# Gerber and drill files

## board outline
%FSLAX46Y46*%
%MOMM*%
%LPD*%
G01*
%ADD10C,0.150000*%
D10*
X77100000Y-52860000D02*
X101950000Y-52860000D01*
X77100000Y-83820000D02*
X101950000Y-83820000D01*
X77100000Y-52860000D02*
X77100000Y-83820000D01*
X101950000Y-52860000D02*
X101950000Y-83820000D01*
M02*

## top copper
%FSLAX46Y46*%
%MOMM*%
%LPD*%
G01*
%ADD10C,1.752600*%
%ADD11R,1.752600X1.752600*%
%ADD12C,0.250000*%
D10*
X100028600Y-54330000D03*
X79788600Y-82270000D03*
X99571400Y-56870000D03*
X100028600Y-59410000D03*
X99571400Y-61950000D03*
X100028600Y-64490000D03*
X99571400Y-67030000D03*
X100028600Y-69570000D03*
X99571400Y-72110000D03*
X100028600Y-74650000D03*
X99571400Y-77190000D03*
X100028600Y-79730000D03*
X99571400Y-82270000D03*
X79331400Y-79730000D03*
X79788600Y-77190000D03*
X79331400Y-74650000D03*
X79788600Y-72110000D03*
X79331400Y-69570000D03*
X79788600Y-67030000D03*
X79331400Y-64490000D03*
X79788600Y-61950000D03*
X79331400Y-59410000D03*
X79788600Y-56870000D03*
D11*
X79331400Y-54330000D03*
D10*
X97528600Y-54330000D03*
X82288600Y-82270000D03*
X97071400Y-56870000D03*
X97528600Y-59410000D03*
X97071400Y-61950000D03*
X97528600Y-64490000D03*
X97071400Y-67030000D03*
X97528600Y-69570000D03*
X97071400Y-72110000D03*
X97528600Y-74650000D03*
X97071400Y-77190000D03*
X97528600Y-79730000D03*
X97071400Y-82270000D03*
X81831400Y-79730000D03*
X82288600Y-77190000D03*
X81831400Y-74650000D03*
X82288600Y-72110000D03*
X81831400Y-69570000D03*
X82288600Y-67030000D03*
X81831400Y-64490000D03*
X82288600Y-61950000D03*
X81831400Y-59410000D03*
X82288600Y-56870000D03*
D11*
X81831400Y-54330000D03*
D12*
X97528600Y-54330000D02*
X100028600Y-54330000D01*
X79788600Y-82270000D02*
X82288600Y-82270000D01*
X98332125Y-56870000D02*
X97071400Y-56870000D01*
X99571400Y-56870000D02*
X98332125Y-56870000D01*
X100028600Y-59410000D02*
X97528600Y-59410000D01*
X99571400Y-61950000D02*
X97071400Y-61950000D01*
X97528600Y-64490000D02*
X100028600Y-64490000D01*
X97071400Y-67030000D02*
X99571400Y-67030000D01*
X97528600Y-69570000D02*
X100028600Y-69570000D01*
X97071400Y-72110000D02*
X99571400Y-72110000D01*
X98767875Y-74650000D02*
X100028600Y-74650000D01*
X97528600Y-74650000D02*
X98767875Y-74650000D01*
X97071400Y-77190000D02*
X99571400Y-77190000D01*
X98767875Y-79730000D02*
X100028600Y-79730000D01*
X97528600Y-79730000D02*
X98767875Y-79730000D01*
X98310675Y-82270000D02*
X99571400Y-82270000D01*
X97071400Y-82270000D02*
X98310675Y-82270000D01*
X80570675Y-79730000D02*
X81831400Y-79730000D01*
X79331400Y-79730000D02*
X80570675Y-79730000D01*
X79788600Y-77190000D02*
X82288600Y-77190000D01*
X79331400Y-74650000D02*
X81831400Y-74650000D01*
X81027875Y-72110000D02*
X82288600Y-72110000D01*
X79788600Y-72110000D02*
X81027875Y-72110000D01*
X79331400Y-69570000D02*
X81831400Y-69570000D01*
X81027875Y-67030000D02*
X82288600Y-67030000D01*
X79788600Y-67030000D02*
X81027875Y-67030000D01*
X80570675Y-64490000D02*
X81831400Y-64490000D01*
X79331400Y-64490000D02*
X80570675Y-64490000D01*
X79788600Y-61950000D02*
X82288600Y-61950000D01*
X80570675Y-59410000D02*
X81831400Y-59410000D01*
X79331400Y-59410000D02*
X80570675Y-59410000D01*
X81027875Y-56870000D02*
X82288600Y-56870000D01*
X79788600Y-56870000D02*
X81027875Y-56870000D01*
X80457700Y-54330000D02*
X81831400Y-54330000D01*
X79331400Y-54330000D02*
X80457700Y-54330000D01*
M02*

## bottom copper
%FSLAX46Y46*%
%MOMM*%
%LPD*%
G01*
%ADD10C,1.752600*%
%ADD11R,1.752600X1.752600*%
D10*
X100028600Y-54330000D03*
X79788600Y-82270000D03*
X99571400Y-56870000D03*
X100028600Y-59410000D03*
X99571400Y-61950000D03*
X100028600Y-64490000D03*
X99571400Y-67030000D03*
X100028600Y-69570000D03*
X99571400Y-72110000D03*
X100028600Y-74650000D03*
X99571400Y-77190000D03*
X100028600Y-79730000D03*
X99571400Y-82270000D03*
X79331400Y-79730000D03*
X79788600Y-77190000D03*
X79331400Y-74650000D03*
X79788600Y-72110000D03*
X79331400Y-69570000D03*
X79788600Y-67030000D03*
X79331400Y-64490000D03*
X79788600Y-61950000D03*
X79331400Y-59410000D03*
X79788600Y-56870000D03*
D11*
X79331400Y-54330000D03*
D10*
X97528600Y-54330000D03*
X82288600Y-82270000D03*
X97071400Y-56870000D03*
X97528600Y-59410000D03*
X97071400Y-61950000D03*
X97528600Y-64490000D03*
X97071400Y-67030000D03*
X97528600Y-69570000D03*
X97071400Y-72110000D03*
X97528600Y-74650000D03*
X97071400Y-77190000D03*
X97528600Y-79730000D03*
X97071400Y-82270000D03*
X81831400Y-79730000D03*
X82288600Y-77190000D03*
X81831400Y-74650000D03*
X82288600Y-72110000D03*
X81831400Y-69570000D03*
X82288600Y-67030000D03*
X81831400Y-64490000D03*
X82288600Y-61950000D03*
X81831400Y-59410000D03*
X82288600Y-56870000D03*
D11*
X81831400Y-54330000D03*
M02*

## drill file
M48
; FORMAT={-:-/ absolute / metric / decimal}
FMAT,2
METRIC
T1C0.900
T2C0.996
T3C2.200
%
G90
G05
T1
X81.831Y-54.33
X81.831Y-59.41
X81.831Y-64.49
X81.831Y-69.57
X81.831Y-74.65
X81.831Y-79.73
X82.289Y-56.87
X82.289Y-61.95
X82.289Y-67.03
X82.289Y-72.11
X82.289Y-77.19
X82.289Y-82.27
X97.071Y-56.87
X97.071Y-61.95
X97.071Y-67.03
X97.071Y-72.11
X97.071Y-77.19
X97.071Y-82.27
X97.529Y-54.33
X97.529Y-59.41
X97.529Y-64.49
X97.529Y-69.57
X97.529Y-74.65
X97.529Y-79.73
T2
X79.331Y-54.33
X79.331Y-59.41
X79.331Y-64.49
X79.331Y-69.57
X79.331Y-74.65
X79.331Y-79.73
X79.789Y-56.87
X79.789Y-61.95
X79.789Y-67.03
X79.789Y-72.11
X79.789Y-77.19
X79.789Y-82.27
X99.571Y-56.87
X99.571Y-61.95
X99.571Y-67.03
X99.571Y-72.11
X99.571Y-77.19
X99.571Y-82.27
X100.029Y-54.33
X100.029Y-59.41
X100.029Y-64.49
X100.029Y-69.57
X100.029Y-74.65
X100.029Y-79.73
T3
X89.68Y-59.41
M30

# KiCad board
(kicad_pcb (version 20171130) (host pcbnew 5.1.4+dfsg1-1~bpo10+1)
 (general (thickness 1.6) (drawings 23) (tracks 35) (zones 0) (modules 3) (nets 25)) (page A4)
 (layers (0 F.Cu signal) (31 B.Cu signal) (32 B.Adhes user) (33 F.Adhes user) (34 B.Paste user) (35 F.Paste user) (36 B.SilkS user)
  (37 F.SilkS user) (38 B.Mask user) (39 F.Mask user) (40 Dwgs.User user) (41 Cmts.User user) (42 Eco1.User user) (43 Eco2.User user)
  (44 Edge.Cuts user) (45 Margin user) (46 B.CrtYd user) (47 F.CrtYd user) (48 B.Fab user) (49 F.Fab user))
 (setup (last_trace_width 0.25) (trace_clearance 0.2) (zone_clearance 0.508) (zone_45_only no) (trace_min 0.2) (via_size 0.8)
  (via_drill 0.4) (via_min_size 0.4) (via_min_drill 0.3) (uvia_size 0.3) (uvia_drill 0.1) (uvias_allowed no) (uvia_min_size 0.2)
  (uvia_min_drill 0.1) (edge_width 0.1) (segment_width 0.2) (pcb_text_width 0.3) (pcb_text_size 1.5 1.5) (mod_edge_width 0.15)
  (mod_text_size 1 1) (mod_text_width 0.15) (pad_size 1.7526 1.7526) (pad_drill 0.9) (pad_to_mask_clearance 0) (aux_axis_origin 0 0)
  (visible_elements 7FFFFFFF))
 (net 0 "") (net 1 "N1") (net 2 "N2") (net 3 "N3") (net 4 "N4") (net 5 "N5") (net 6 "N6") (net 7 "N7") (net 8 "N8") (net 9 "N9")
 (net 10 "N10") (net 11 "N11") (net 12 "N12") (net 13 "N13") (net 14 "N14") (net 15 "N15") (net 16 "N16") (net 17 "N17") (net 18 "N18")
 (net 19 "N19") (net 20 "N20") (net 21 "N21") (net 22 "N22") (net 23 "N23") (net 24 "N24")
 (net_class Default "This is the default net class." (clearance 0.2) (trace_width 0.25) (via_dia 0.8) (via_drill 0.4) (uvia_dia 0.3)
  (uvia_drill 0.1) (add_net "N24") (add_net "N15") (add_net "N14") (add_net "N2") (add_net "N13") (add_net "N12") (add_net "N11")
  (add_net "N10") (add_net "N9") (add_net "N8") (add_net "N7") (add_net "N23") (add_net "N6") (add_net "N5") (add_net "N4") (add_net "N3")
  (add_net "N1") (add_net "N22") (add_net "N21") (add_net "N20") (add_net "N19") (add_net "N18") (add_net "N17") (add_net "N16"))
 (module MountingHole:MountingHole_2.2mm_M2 (layer F.Cu) (at 89.68 59.41)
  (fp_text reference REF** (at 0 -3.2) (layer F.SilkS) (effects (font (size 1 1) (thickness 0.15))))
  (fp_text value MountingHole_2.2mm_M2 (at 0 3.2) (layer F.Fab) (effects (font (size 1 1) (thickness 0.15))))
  (pad 1 np_thru_hole circle (at 0 0) (size 2.2 2.2) (drill 2.2) (layers *.Cu *.Mask)))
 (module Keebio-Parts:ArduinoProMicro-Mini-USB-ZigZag (layer F.Cu) (at 89.68 68.3 270)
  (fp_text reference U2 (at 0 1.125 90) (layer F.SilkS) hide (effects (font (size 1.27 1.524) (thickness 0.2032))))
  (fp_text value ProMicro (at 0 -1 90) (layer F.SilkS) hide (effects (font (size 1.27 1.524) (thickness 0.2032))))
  (pad 24 thru_hole circle (at -13.97 -10.3486 270) (size 1.7526 1.7526) (drill 0.9961) (layers *.Cu *.SilkS *.Mask) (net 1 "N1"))
  (pad 12 thru_hole circle (at 13.97 9.8914 270) (size 1.7526 1.7526) (drill 0.9961) (layers *.Cu *.SilkS *.Mask) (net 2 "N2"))
  (pad 23 thru_hole circle (at -11.43 -9.8914 270) (size 1.7526 1.7526) (drill 0.9961) (layers *.Cu *.SilkS *.Mask) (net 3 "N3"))
  (pad 22 thru_hole circle (at -8.89 -10.3486 270) (size 1.7526 1.7526) (drill 0.9961) (layers *.Cu *.SilkS *.Mask) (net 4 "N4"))
  (pad 21 thru_hole circle (at -6.35 -9.8914 270) (size 1.7526 1.7526) (drill 0.9961) (layers *.Cu *.SilkS *.Mask) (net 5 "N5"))
  (pad 20 thru_hole circle (at -3.81 -10.3486 270) (size 1.7526 1.7526) (drill 0.9961) (layers *.Cu *.SilkS *.Mask) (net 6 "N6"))
  (pad 19 thru_hole circle (at -1.27 -9.8914 270) (size 1.7526 1.7526) (drill 0.9961) (layers *.Cu *.SilkS *.Mask) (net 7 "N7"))
  (pad 18 thru_hole circle (at 1.27 -10.3486 270) (size 1.7526 1.7526) (drill 0.9961) (layers *.Cu *.SilkS *.Mask) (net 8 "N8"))
  (pad 17 thru_hole circle (at 3.81 -9.8914 270) (size 1.7526 1.7526) (drill 0.9961) (layers *.Cu *.SilkS *.Mask) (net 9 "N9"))
  (pad 16 thru_hole circle (at 6.35 -10.3486 270) (size 1.7526 1.7526) (drill 0.9961) (layers *.Cu *.SilkS *.Mask) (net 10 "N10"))
  (pad 15 thru_hole circle (at 8.89 -9.8914 270) (size 1.7526 1.7526) (drill 0.9961) (layers *.Cu *.SilkS *.Mask) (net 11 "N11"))
  (pad 14 thru_hole circle (at 11.43 -10.3486 270) (size 1.7526 1.7526) (drill 0.9961) (layers *.Cu *.SilkS *.Mask) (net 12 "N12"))
  (pad 13 thru_hole circle (at 13.97 -9.8914 270) (size 1.7526 1.7526) (drill 0.9961) (layers *.Cu *.SilkS *.Mask) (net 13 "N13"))
  (pad 11 thru_hole circle (at 11.43 10.3486 270) (size 1.7526 1.7526) (drill 0.9961) (layers *.Cu *.SilkS *.Mask) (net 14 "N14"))
  (pad 10 thru_hole circle (at 8.89 9.8914 270) (size 1.7526 1.7526) (drill 0.9961) (layers *.Cu *.SilkS *.Mask) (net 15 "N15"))
  (pad 9 thru_hole circle (at 6.35 10.3486 270) (size 1.7526 1.7526) (drill 0.9961) (layers *.Cu *.SilkS *.Mask) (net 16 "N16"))
  (pad 8 thru_hole circle (at 3.81 9.8914 270) (size 1.7526 1.7526) (drill 0.9961) (layers *.Cu *.SilkS *.Mask) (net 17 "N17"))
  (pad 7 thru_hole circle (at 1.27 10.3486 270) (size 1.7526 1.7526) (drill 0.9961) (layers *.Cu *.SilkS *.Mask) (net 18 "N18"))
  (pad 6 thru_hole circle (at -1.27 9.8914 270) (size 1.7526 1.7526) (drill 0.9961) (layers *.Cu *.SilkS *.Mask) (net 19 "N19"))
  (pad 5 thru_hole circle (at -3.81 10.3486 270) (size 1.7526 1.7526) (drill 0.9961) (layers *.Cu *.SilkS *.Mask) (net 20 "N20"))
  (pad 4 thru_hole circle (at -6.35 9.8914 270) (size 1.7526 1.7526) (drill 0.9961) (layers *.Cu *.SilkS *.Mask) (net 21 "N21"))
  (pad 3 thru_hole circle (at -8.89 10.3486 270) (size 1.7526 1.7526) (drill 0.9961) (layers *.Cu *.SilkS *.Mask) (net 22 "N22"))
  (pad 2 thru_hole circle (at -11.43 9.8914 270) (size 1.7526 1.7526) (drill 0.9961) (layers *.Cu *.SilkS *.Mask) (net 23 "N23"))
  (pad 1 thru_hole rect (at -13.97 10.3486 270) (size 1.7526 1.7526) (drill 0.9961) (layers *.Cu *.SilkS *.Mask) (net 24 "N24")))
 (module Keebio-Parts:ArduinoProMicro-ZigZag (layer F.Cu) (at 89.68 68.3 270)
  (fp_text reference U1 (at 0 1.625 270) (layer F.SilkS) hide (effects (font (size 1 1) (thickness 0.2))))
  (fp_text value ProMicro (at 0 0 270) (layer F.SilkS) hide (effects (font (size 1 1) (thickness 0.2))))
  (pad 24 thru_hole circle (at -13.97 -7.8486 270) (size 1.7526 1.7526) (drill 0.9) (layers *.Cu *.SilkS *.Mask) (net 1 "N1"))
  (pad 12 thru_hole circle (at 13.97 7.3914 270) (size 1.7526 1.7526) (drill 0.9) (layers *.Cu *.SilkS *.Mask) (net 2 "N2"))
  (pad 23 thru_hole circle (at -11.43 -7.3914 270) (size 1.7526 1.7526) (drill 0.9) (layers *.Cu *.SilkS *.Mask) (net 3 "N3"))
  (pad 22 thru_hole circle (at -8.89 -7.8486 270) (size 1.7526 1.7526) (drill 0.9) (layers *.Cu *.SilkS *.Mask) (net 4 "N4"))
  (pad 21 thru_hole circle (at -6.35 -7.3914 270) (size 1.7526 1.7526) (drill 0.9) (layers *.Cu *.SilkS *.Mask) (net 5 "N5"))
  (pad 20 thru_hole circle (at -3.81 -7.8486 270) (size 1.7526 1.7526) (drill 0.9) (layers *.Cu *.SilkS *.Mask) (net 6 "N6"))
  (pad 19 thru_hole circle (at -1.27 -7.3914 270) (size 1.7526 1.7526) (drill 0.9) (layers *.Cu *.SilkS *.Mask) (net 7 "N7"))
  (pad 18 thru_hole circle (at 1.27 -7.8486 270) (size 1.7526 1.7526) (drill 0.9) (layers *.Cu *.SilkS *.Mask) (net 8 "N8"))
  (pad 17 thru_hole circle (at 3.81 -7.3914 270) (size 1.7526 1.7526) (drill 0.9) (layers *.Cu *.SilkS *.Mask) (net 9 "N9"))
  (pad 16 thru_hole circle (at 6.35 -7.8486 270) (size 1.7526 1.7526) (drill 0.9) (layers *.Cu *.SilkS *.Mask) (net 10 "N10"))
  (pad 15 thru_hole circle (at 8.89 -7.3914 270) (size 1.7526 1.7526) (drill 0.9) (layers *.Cu *.SilkS *.Mask) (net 11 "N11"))
  (pad 14 thru_hole circle (at 11.43 -7.8486 270) (size 1.7526 1.7526) (drill 0.9) (layers *.Cu *.SilkS *.Mask) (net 12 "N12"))
  (pad 13 thru_hole circle (at 13.97 -7.3914 270) (size 1.7526 1.7526) (drill 0.9) (layers *.Cu *.SilkS *.Mask) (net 13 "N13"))
  (pad 11 thru_hole circle (at 11.43 7.8486 270) (size 1.7526 1.7526) (drill 0.9) (layers *.Cu *.SilkS *.Mask) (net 14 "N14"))
  (pad 10 thru_hole circle (at 8.89 7.3914 270) (size 1.7526 1.7526) (drill 0.9) (layers *.Cu *.SilkS *.Mask) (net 15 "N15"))
  (pad 9 thru_hole circle (at 6.35 7.8486 270) (size 1.7526 1.7526) (drill 0.9) (layers *.Cu *.SilkS *.Mask) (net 16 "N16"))
  (pad 8 thru_hole circle (at 3.81 7.3914 270) (size 1.7526 1.7526) (drill 0.9) (layers *.Cu *.SilkS *.Mask) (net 17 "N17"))
  (pad 7 thru_hole circle (at 1.27 7.8486 270) (size 1.7526 1.7526) (drill 0.9) (layers *.Cu *.SilkS *.Mask) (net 18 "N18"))
  (pad 6 thru_hole circle (at -1.27 7.3914 270) (size 1.7526 1.7526) (drill 0.9) (layers *.Cu *.SilkS *.Mask) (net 19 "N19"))
  (pad 5 thru_hole circle (at -3.81 7.8486 270) (size 1.7526 1.7526) (drill 0.9) (layers *.Cu *.SilkS *.Mask) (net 20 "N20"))
  (pad 4 thru_hole circle (at -6.35 7.3914 270) (size 1.7526 1.7526) (drill 0.9) (layers *.Cu *.SilkS *.Mask) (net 21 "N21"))
  (pad 3 thru_hole circle (at -8.89 7.8486 270) (size 1.7526 1.7526) (drill 0.9) (layers *.Cu *.SilkS *.Mask) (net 22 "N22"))
  (pad 2 thru_hole circle (at -11.43 7.3914 270) (size 1.7526 1.7526) (drill 0.9) (layers *.Cu *.SilkS *.Mask) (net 23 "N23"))
  (pad 1 thru_hole rect (at -13.97 7.8486 270) (size 1.7526 1.7526) (drill 0.9) (layers *.Cu *.SilkS *.Mask) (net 24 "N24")))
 (gr_line (start 77.1 52.86) (end 101.95 52.86) (layer Edge.Cuts) (width 0.15))
 (gr_line (start 77.1 83.82) (end 101.95 83.82) (layer Edge.Cuts) (width 0.15))
 (gr_line (start 77.1 52.86) (end 77.1 83.82) (layer Edge.Cuts) (width 0.15))
 (gr_line (start 101.95 52.86) (end 101.95 83.82) (layer Edge.Cuts) (width 0.15))
 (segment (start 97.5286 54.33) (end 100.0286 54.33) (width 0.25) (layer F.Cu) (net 1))
 (segment (start 79.7886 82.27) (end 82.2886 82.27) (width 0.25) (layer F.Cu) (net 2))
 (segment (start 98.332125 56.87) (end 97.0714 56.87) (width 0.25) (layer F.Cu) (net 3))
 (segment (start 99.5714 56.87) (end 98.332125 56.87) (width 0.25) (layer F.Cu) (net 3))
 (segment (start 100.0286 59.41) (end 97.5286 59.41) (width 0.25) (layer F.Cu) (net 4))
 (segment (start 99.5714 61.95) (end 97.0714 61.95) (width 0.25) (layer F.Cu) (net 5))
 (segment (start 97.5286 64.49) (end 100.0286 64.49) (width 0.25) (layer F.Cu) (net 6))
 (segment (start 97.0714 67.03) (end 99.5714 67.03) (width 0.25) (layer F.Cu) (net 7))
 (segment (start 97.5286 69.57) (end 100.0286 69.57) (width 0.25) (layer F.Cu) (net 8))
 (segment (start 97.0714 72.11) (end 99.5714 72.11) (width 0.25) (layer F.Cu) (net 9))
 (segment (start 98.767875 74.65) (end 100.0286 74.65) (width 0.25) (layer F.Cu) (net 10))
 (segment (start 97.5286 74.65) (end 98.767875 74.65) (width 0.25) (layer F.Cu) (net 10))
 (segment (start 97.0714 77.19) (end 99.5714 77.19) (width 0.25) (layer F.Cu) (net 11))
 (segment (start 98.767875 79.73) (end 100.0286 79.73) (width 0.25) (layer F.Cu) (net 12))
 (segment (start 97.5286 79.73) (end 98.767875 79.73) (width 0.25) (layer F.Cu) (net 12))
 (segment (start 98.310675 82.27) (end 99.5714 82.27) (width 0.25) (layer F.Cu) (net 13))
 (segment (start 97.0714 82.27) (end 98.310675 82.27) (width 0.25) (layer F.Cu) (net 13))
 (segment (start 80.570675 79.73) (end 81.8314 79.73) (width 0.25) (layer F.Cu) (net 14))
 (segment (start 79.3314 79.73) (end 80.570675 79.73) (width 0.25) (layer F.Cu) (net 14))
 (segment (start 79.7886 77.19) (end 82.2886 77.19) (width 0.25) (layer F.Cu) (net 15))
 (segment (start 79.3314 74.65) (end 81.8314 74.65) (width 0.25) (layer F.Cu) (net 16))
 (segment (start 81.027875 72.11) (end 82.2886 72.11) (width 0.25) (layer F.Cu) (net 17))
 (segment (start 79.7886 72.11) (end 81.027875 72.11) (width 0.25) (layer F.Cu) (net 17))
 (segment (start 79.3314 69.57) (end 81.8314 69.57) (width 0.25) (layer F.Cu) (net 18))
 (segment (start 81.027875 67.03) (end 82.2886 67.03) (width 0.25) (layer F.Cu) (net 19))
 (segment (start 79.7886 67.03) (end 81.027875 67.03) (width 0.25) (layer F.Cu) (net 19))
 (segment (start 80.570675 64.49) (end 81.8314 64.49) (width 0.25) (layer F.Cu) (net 20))
 (segment (start 79.3314 64.49) (end 80.570675 64.49) (width 0.25) (layer F.Cu) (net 20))
 (segment (start 79.7886 61.95) (end 82.2886 61.95) (width 0.25) (layer F.Cu) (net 21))
 (segment (start 80.570675 59.41) (end 81.8314 59.41) (width 0.25) (layer F.Cu) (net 22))
 (segment (start 79.3314 59.41) (end 80.570675 59.41) (width 0.25) (layer F.Cu) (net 22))
 (segment (start 81.027875 56.87) (end 82.2886 56.87) (width 0.25) (layer F.Cu) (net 23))
 (segment (start 79.7886 56.87) (end 81.027875 56.87) (width 0.25) (layer F.Cu) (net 23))
 (segment (start 80.4577 54.33) (end 81.8314 54.33) (width 0.25) (layer F.Cu) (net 24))
 (segment (start 79.3314 54.33) (end 80.4577 54.33) (width 0.25) (layer F.Cu) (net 24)))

